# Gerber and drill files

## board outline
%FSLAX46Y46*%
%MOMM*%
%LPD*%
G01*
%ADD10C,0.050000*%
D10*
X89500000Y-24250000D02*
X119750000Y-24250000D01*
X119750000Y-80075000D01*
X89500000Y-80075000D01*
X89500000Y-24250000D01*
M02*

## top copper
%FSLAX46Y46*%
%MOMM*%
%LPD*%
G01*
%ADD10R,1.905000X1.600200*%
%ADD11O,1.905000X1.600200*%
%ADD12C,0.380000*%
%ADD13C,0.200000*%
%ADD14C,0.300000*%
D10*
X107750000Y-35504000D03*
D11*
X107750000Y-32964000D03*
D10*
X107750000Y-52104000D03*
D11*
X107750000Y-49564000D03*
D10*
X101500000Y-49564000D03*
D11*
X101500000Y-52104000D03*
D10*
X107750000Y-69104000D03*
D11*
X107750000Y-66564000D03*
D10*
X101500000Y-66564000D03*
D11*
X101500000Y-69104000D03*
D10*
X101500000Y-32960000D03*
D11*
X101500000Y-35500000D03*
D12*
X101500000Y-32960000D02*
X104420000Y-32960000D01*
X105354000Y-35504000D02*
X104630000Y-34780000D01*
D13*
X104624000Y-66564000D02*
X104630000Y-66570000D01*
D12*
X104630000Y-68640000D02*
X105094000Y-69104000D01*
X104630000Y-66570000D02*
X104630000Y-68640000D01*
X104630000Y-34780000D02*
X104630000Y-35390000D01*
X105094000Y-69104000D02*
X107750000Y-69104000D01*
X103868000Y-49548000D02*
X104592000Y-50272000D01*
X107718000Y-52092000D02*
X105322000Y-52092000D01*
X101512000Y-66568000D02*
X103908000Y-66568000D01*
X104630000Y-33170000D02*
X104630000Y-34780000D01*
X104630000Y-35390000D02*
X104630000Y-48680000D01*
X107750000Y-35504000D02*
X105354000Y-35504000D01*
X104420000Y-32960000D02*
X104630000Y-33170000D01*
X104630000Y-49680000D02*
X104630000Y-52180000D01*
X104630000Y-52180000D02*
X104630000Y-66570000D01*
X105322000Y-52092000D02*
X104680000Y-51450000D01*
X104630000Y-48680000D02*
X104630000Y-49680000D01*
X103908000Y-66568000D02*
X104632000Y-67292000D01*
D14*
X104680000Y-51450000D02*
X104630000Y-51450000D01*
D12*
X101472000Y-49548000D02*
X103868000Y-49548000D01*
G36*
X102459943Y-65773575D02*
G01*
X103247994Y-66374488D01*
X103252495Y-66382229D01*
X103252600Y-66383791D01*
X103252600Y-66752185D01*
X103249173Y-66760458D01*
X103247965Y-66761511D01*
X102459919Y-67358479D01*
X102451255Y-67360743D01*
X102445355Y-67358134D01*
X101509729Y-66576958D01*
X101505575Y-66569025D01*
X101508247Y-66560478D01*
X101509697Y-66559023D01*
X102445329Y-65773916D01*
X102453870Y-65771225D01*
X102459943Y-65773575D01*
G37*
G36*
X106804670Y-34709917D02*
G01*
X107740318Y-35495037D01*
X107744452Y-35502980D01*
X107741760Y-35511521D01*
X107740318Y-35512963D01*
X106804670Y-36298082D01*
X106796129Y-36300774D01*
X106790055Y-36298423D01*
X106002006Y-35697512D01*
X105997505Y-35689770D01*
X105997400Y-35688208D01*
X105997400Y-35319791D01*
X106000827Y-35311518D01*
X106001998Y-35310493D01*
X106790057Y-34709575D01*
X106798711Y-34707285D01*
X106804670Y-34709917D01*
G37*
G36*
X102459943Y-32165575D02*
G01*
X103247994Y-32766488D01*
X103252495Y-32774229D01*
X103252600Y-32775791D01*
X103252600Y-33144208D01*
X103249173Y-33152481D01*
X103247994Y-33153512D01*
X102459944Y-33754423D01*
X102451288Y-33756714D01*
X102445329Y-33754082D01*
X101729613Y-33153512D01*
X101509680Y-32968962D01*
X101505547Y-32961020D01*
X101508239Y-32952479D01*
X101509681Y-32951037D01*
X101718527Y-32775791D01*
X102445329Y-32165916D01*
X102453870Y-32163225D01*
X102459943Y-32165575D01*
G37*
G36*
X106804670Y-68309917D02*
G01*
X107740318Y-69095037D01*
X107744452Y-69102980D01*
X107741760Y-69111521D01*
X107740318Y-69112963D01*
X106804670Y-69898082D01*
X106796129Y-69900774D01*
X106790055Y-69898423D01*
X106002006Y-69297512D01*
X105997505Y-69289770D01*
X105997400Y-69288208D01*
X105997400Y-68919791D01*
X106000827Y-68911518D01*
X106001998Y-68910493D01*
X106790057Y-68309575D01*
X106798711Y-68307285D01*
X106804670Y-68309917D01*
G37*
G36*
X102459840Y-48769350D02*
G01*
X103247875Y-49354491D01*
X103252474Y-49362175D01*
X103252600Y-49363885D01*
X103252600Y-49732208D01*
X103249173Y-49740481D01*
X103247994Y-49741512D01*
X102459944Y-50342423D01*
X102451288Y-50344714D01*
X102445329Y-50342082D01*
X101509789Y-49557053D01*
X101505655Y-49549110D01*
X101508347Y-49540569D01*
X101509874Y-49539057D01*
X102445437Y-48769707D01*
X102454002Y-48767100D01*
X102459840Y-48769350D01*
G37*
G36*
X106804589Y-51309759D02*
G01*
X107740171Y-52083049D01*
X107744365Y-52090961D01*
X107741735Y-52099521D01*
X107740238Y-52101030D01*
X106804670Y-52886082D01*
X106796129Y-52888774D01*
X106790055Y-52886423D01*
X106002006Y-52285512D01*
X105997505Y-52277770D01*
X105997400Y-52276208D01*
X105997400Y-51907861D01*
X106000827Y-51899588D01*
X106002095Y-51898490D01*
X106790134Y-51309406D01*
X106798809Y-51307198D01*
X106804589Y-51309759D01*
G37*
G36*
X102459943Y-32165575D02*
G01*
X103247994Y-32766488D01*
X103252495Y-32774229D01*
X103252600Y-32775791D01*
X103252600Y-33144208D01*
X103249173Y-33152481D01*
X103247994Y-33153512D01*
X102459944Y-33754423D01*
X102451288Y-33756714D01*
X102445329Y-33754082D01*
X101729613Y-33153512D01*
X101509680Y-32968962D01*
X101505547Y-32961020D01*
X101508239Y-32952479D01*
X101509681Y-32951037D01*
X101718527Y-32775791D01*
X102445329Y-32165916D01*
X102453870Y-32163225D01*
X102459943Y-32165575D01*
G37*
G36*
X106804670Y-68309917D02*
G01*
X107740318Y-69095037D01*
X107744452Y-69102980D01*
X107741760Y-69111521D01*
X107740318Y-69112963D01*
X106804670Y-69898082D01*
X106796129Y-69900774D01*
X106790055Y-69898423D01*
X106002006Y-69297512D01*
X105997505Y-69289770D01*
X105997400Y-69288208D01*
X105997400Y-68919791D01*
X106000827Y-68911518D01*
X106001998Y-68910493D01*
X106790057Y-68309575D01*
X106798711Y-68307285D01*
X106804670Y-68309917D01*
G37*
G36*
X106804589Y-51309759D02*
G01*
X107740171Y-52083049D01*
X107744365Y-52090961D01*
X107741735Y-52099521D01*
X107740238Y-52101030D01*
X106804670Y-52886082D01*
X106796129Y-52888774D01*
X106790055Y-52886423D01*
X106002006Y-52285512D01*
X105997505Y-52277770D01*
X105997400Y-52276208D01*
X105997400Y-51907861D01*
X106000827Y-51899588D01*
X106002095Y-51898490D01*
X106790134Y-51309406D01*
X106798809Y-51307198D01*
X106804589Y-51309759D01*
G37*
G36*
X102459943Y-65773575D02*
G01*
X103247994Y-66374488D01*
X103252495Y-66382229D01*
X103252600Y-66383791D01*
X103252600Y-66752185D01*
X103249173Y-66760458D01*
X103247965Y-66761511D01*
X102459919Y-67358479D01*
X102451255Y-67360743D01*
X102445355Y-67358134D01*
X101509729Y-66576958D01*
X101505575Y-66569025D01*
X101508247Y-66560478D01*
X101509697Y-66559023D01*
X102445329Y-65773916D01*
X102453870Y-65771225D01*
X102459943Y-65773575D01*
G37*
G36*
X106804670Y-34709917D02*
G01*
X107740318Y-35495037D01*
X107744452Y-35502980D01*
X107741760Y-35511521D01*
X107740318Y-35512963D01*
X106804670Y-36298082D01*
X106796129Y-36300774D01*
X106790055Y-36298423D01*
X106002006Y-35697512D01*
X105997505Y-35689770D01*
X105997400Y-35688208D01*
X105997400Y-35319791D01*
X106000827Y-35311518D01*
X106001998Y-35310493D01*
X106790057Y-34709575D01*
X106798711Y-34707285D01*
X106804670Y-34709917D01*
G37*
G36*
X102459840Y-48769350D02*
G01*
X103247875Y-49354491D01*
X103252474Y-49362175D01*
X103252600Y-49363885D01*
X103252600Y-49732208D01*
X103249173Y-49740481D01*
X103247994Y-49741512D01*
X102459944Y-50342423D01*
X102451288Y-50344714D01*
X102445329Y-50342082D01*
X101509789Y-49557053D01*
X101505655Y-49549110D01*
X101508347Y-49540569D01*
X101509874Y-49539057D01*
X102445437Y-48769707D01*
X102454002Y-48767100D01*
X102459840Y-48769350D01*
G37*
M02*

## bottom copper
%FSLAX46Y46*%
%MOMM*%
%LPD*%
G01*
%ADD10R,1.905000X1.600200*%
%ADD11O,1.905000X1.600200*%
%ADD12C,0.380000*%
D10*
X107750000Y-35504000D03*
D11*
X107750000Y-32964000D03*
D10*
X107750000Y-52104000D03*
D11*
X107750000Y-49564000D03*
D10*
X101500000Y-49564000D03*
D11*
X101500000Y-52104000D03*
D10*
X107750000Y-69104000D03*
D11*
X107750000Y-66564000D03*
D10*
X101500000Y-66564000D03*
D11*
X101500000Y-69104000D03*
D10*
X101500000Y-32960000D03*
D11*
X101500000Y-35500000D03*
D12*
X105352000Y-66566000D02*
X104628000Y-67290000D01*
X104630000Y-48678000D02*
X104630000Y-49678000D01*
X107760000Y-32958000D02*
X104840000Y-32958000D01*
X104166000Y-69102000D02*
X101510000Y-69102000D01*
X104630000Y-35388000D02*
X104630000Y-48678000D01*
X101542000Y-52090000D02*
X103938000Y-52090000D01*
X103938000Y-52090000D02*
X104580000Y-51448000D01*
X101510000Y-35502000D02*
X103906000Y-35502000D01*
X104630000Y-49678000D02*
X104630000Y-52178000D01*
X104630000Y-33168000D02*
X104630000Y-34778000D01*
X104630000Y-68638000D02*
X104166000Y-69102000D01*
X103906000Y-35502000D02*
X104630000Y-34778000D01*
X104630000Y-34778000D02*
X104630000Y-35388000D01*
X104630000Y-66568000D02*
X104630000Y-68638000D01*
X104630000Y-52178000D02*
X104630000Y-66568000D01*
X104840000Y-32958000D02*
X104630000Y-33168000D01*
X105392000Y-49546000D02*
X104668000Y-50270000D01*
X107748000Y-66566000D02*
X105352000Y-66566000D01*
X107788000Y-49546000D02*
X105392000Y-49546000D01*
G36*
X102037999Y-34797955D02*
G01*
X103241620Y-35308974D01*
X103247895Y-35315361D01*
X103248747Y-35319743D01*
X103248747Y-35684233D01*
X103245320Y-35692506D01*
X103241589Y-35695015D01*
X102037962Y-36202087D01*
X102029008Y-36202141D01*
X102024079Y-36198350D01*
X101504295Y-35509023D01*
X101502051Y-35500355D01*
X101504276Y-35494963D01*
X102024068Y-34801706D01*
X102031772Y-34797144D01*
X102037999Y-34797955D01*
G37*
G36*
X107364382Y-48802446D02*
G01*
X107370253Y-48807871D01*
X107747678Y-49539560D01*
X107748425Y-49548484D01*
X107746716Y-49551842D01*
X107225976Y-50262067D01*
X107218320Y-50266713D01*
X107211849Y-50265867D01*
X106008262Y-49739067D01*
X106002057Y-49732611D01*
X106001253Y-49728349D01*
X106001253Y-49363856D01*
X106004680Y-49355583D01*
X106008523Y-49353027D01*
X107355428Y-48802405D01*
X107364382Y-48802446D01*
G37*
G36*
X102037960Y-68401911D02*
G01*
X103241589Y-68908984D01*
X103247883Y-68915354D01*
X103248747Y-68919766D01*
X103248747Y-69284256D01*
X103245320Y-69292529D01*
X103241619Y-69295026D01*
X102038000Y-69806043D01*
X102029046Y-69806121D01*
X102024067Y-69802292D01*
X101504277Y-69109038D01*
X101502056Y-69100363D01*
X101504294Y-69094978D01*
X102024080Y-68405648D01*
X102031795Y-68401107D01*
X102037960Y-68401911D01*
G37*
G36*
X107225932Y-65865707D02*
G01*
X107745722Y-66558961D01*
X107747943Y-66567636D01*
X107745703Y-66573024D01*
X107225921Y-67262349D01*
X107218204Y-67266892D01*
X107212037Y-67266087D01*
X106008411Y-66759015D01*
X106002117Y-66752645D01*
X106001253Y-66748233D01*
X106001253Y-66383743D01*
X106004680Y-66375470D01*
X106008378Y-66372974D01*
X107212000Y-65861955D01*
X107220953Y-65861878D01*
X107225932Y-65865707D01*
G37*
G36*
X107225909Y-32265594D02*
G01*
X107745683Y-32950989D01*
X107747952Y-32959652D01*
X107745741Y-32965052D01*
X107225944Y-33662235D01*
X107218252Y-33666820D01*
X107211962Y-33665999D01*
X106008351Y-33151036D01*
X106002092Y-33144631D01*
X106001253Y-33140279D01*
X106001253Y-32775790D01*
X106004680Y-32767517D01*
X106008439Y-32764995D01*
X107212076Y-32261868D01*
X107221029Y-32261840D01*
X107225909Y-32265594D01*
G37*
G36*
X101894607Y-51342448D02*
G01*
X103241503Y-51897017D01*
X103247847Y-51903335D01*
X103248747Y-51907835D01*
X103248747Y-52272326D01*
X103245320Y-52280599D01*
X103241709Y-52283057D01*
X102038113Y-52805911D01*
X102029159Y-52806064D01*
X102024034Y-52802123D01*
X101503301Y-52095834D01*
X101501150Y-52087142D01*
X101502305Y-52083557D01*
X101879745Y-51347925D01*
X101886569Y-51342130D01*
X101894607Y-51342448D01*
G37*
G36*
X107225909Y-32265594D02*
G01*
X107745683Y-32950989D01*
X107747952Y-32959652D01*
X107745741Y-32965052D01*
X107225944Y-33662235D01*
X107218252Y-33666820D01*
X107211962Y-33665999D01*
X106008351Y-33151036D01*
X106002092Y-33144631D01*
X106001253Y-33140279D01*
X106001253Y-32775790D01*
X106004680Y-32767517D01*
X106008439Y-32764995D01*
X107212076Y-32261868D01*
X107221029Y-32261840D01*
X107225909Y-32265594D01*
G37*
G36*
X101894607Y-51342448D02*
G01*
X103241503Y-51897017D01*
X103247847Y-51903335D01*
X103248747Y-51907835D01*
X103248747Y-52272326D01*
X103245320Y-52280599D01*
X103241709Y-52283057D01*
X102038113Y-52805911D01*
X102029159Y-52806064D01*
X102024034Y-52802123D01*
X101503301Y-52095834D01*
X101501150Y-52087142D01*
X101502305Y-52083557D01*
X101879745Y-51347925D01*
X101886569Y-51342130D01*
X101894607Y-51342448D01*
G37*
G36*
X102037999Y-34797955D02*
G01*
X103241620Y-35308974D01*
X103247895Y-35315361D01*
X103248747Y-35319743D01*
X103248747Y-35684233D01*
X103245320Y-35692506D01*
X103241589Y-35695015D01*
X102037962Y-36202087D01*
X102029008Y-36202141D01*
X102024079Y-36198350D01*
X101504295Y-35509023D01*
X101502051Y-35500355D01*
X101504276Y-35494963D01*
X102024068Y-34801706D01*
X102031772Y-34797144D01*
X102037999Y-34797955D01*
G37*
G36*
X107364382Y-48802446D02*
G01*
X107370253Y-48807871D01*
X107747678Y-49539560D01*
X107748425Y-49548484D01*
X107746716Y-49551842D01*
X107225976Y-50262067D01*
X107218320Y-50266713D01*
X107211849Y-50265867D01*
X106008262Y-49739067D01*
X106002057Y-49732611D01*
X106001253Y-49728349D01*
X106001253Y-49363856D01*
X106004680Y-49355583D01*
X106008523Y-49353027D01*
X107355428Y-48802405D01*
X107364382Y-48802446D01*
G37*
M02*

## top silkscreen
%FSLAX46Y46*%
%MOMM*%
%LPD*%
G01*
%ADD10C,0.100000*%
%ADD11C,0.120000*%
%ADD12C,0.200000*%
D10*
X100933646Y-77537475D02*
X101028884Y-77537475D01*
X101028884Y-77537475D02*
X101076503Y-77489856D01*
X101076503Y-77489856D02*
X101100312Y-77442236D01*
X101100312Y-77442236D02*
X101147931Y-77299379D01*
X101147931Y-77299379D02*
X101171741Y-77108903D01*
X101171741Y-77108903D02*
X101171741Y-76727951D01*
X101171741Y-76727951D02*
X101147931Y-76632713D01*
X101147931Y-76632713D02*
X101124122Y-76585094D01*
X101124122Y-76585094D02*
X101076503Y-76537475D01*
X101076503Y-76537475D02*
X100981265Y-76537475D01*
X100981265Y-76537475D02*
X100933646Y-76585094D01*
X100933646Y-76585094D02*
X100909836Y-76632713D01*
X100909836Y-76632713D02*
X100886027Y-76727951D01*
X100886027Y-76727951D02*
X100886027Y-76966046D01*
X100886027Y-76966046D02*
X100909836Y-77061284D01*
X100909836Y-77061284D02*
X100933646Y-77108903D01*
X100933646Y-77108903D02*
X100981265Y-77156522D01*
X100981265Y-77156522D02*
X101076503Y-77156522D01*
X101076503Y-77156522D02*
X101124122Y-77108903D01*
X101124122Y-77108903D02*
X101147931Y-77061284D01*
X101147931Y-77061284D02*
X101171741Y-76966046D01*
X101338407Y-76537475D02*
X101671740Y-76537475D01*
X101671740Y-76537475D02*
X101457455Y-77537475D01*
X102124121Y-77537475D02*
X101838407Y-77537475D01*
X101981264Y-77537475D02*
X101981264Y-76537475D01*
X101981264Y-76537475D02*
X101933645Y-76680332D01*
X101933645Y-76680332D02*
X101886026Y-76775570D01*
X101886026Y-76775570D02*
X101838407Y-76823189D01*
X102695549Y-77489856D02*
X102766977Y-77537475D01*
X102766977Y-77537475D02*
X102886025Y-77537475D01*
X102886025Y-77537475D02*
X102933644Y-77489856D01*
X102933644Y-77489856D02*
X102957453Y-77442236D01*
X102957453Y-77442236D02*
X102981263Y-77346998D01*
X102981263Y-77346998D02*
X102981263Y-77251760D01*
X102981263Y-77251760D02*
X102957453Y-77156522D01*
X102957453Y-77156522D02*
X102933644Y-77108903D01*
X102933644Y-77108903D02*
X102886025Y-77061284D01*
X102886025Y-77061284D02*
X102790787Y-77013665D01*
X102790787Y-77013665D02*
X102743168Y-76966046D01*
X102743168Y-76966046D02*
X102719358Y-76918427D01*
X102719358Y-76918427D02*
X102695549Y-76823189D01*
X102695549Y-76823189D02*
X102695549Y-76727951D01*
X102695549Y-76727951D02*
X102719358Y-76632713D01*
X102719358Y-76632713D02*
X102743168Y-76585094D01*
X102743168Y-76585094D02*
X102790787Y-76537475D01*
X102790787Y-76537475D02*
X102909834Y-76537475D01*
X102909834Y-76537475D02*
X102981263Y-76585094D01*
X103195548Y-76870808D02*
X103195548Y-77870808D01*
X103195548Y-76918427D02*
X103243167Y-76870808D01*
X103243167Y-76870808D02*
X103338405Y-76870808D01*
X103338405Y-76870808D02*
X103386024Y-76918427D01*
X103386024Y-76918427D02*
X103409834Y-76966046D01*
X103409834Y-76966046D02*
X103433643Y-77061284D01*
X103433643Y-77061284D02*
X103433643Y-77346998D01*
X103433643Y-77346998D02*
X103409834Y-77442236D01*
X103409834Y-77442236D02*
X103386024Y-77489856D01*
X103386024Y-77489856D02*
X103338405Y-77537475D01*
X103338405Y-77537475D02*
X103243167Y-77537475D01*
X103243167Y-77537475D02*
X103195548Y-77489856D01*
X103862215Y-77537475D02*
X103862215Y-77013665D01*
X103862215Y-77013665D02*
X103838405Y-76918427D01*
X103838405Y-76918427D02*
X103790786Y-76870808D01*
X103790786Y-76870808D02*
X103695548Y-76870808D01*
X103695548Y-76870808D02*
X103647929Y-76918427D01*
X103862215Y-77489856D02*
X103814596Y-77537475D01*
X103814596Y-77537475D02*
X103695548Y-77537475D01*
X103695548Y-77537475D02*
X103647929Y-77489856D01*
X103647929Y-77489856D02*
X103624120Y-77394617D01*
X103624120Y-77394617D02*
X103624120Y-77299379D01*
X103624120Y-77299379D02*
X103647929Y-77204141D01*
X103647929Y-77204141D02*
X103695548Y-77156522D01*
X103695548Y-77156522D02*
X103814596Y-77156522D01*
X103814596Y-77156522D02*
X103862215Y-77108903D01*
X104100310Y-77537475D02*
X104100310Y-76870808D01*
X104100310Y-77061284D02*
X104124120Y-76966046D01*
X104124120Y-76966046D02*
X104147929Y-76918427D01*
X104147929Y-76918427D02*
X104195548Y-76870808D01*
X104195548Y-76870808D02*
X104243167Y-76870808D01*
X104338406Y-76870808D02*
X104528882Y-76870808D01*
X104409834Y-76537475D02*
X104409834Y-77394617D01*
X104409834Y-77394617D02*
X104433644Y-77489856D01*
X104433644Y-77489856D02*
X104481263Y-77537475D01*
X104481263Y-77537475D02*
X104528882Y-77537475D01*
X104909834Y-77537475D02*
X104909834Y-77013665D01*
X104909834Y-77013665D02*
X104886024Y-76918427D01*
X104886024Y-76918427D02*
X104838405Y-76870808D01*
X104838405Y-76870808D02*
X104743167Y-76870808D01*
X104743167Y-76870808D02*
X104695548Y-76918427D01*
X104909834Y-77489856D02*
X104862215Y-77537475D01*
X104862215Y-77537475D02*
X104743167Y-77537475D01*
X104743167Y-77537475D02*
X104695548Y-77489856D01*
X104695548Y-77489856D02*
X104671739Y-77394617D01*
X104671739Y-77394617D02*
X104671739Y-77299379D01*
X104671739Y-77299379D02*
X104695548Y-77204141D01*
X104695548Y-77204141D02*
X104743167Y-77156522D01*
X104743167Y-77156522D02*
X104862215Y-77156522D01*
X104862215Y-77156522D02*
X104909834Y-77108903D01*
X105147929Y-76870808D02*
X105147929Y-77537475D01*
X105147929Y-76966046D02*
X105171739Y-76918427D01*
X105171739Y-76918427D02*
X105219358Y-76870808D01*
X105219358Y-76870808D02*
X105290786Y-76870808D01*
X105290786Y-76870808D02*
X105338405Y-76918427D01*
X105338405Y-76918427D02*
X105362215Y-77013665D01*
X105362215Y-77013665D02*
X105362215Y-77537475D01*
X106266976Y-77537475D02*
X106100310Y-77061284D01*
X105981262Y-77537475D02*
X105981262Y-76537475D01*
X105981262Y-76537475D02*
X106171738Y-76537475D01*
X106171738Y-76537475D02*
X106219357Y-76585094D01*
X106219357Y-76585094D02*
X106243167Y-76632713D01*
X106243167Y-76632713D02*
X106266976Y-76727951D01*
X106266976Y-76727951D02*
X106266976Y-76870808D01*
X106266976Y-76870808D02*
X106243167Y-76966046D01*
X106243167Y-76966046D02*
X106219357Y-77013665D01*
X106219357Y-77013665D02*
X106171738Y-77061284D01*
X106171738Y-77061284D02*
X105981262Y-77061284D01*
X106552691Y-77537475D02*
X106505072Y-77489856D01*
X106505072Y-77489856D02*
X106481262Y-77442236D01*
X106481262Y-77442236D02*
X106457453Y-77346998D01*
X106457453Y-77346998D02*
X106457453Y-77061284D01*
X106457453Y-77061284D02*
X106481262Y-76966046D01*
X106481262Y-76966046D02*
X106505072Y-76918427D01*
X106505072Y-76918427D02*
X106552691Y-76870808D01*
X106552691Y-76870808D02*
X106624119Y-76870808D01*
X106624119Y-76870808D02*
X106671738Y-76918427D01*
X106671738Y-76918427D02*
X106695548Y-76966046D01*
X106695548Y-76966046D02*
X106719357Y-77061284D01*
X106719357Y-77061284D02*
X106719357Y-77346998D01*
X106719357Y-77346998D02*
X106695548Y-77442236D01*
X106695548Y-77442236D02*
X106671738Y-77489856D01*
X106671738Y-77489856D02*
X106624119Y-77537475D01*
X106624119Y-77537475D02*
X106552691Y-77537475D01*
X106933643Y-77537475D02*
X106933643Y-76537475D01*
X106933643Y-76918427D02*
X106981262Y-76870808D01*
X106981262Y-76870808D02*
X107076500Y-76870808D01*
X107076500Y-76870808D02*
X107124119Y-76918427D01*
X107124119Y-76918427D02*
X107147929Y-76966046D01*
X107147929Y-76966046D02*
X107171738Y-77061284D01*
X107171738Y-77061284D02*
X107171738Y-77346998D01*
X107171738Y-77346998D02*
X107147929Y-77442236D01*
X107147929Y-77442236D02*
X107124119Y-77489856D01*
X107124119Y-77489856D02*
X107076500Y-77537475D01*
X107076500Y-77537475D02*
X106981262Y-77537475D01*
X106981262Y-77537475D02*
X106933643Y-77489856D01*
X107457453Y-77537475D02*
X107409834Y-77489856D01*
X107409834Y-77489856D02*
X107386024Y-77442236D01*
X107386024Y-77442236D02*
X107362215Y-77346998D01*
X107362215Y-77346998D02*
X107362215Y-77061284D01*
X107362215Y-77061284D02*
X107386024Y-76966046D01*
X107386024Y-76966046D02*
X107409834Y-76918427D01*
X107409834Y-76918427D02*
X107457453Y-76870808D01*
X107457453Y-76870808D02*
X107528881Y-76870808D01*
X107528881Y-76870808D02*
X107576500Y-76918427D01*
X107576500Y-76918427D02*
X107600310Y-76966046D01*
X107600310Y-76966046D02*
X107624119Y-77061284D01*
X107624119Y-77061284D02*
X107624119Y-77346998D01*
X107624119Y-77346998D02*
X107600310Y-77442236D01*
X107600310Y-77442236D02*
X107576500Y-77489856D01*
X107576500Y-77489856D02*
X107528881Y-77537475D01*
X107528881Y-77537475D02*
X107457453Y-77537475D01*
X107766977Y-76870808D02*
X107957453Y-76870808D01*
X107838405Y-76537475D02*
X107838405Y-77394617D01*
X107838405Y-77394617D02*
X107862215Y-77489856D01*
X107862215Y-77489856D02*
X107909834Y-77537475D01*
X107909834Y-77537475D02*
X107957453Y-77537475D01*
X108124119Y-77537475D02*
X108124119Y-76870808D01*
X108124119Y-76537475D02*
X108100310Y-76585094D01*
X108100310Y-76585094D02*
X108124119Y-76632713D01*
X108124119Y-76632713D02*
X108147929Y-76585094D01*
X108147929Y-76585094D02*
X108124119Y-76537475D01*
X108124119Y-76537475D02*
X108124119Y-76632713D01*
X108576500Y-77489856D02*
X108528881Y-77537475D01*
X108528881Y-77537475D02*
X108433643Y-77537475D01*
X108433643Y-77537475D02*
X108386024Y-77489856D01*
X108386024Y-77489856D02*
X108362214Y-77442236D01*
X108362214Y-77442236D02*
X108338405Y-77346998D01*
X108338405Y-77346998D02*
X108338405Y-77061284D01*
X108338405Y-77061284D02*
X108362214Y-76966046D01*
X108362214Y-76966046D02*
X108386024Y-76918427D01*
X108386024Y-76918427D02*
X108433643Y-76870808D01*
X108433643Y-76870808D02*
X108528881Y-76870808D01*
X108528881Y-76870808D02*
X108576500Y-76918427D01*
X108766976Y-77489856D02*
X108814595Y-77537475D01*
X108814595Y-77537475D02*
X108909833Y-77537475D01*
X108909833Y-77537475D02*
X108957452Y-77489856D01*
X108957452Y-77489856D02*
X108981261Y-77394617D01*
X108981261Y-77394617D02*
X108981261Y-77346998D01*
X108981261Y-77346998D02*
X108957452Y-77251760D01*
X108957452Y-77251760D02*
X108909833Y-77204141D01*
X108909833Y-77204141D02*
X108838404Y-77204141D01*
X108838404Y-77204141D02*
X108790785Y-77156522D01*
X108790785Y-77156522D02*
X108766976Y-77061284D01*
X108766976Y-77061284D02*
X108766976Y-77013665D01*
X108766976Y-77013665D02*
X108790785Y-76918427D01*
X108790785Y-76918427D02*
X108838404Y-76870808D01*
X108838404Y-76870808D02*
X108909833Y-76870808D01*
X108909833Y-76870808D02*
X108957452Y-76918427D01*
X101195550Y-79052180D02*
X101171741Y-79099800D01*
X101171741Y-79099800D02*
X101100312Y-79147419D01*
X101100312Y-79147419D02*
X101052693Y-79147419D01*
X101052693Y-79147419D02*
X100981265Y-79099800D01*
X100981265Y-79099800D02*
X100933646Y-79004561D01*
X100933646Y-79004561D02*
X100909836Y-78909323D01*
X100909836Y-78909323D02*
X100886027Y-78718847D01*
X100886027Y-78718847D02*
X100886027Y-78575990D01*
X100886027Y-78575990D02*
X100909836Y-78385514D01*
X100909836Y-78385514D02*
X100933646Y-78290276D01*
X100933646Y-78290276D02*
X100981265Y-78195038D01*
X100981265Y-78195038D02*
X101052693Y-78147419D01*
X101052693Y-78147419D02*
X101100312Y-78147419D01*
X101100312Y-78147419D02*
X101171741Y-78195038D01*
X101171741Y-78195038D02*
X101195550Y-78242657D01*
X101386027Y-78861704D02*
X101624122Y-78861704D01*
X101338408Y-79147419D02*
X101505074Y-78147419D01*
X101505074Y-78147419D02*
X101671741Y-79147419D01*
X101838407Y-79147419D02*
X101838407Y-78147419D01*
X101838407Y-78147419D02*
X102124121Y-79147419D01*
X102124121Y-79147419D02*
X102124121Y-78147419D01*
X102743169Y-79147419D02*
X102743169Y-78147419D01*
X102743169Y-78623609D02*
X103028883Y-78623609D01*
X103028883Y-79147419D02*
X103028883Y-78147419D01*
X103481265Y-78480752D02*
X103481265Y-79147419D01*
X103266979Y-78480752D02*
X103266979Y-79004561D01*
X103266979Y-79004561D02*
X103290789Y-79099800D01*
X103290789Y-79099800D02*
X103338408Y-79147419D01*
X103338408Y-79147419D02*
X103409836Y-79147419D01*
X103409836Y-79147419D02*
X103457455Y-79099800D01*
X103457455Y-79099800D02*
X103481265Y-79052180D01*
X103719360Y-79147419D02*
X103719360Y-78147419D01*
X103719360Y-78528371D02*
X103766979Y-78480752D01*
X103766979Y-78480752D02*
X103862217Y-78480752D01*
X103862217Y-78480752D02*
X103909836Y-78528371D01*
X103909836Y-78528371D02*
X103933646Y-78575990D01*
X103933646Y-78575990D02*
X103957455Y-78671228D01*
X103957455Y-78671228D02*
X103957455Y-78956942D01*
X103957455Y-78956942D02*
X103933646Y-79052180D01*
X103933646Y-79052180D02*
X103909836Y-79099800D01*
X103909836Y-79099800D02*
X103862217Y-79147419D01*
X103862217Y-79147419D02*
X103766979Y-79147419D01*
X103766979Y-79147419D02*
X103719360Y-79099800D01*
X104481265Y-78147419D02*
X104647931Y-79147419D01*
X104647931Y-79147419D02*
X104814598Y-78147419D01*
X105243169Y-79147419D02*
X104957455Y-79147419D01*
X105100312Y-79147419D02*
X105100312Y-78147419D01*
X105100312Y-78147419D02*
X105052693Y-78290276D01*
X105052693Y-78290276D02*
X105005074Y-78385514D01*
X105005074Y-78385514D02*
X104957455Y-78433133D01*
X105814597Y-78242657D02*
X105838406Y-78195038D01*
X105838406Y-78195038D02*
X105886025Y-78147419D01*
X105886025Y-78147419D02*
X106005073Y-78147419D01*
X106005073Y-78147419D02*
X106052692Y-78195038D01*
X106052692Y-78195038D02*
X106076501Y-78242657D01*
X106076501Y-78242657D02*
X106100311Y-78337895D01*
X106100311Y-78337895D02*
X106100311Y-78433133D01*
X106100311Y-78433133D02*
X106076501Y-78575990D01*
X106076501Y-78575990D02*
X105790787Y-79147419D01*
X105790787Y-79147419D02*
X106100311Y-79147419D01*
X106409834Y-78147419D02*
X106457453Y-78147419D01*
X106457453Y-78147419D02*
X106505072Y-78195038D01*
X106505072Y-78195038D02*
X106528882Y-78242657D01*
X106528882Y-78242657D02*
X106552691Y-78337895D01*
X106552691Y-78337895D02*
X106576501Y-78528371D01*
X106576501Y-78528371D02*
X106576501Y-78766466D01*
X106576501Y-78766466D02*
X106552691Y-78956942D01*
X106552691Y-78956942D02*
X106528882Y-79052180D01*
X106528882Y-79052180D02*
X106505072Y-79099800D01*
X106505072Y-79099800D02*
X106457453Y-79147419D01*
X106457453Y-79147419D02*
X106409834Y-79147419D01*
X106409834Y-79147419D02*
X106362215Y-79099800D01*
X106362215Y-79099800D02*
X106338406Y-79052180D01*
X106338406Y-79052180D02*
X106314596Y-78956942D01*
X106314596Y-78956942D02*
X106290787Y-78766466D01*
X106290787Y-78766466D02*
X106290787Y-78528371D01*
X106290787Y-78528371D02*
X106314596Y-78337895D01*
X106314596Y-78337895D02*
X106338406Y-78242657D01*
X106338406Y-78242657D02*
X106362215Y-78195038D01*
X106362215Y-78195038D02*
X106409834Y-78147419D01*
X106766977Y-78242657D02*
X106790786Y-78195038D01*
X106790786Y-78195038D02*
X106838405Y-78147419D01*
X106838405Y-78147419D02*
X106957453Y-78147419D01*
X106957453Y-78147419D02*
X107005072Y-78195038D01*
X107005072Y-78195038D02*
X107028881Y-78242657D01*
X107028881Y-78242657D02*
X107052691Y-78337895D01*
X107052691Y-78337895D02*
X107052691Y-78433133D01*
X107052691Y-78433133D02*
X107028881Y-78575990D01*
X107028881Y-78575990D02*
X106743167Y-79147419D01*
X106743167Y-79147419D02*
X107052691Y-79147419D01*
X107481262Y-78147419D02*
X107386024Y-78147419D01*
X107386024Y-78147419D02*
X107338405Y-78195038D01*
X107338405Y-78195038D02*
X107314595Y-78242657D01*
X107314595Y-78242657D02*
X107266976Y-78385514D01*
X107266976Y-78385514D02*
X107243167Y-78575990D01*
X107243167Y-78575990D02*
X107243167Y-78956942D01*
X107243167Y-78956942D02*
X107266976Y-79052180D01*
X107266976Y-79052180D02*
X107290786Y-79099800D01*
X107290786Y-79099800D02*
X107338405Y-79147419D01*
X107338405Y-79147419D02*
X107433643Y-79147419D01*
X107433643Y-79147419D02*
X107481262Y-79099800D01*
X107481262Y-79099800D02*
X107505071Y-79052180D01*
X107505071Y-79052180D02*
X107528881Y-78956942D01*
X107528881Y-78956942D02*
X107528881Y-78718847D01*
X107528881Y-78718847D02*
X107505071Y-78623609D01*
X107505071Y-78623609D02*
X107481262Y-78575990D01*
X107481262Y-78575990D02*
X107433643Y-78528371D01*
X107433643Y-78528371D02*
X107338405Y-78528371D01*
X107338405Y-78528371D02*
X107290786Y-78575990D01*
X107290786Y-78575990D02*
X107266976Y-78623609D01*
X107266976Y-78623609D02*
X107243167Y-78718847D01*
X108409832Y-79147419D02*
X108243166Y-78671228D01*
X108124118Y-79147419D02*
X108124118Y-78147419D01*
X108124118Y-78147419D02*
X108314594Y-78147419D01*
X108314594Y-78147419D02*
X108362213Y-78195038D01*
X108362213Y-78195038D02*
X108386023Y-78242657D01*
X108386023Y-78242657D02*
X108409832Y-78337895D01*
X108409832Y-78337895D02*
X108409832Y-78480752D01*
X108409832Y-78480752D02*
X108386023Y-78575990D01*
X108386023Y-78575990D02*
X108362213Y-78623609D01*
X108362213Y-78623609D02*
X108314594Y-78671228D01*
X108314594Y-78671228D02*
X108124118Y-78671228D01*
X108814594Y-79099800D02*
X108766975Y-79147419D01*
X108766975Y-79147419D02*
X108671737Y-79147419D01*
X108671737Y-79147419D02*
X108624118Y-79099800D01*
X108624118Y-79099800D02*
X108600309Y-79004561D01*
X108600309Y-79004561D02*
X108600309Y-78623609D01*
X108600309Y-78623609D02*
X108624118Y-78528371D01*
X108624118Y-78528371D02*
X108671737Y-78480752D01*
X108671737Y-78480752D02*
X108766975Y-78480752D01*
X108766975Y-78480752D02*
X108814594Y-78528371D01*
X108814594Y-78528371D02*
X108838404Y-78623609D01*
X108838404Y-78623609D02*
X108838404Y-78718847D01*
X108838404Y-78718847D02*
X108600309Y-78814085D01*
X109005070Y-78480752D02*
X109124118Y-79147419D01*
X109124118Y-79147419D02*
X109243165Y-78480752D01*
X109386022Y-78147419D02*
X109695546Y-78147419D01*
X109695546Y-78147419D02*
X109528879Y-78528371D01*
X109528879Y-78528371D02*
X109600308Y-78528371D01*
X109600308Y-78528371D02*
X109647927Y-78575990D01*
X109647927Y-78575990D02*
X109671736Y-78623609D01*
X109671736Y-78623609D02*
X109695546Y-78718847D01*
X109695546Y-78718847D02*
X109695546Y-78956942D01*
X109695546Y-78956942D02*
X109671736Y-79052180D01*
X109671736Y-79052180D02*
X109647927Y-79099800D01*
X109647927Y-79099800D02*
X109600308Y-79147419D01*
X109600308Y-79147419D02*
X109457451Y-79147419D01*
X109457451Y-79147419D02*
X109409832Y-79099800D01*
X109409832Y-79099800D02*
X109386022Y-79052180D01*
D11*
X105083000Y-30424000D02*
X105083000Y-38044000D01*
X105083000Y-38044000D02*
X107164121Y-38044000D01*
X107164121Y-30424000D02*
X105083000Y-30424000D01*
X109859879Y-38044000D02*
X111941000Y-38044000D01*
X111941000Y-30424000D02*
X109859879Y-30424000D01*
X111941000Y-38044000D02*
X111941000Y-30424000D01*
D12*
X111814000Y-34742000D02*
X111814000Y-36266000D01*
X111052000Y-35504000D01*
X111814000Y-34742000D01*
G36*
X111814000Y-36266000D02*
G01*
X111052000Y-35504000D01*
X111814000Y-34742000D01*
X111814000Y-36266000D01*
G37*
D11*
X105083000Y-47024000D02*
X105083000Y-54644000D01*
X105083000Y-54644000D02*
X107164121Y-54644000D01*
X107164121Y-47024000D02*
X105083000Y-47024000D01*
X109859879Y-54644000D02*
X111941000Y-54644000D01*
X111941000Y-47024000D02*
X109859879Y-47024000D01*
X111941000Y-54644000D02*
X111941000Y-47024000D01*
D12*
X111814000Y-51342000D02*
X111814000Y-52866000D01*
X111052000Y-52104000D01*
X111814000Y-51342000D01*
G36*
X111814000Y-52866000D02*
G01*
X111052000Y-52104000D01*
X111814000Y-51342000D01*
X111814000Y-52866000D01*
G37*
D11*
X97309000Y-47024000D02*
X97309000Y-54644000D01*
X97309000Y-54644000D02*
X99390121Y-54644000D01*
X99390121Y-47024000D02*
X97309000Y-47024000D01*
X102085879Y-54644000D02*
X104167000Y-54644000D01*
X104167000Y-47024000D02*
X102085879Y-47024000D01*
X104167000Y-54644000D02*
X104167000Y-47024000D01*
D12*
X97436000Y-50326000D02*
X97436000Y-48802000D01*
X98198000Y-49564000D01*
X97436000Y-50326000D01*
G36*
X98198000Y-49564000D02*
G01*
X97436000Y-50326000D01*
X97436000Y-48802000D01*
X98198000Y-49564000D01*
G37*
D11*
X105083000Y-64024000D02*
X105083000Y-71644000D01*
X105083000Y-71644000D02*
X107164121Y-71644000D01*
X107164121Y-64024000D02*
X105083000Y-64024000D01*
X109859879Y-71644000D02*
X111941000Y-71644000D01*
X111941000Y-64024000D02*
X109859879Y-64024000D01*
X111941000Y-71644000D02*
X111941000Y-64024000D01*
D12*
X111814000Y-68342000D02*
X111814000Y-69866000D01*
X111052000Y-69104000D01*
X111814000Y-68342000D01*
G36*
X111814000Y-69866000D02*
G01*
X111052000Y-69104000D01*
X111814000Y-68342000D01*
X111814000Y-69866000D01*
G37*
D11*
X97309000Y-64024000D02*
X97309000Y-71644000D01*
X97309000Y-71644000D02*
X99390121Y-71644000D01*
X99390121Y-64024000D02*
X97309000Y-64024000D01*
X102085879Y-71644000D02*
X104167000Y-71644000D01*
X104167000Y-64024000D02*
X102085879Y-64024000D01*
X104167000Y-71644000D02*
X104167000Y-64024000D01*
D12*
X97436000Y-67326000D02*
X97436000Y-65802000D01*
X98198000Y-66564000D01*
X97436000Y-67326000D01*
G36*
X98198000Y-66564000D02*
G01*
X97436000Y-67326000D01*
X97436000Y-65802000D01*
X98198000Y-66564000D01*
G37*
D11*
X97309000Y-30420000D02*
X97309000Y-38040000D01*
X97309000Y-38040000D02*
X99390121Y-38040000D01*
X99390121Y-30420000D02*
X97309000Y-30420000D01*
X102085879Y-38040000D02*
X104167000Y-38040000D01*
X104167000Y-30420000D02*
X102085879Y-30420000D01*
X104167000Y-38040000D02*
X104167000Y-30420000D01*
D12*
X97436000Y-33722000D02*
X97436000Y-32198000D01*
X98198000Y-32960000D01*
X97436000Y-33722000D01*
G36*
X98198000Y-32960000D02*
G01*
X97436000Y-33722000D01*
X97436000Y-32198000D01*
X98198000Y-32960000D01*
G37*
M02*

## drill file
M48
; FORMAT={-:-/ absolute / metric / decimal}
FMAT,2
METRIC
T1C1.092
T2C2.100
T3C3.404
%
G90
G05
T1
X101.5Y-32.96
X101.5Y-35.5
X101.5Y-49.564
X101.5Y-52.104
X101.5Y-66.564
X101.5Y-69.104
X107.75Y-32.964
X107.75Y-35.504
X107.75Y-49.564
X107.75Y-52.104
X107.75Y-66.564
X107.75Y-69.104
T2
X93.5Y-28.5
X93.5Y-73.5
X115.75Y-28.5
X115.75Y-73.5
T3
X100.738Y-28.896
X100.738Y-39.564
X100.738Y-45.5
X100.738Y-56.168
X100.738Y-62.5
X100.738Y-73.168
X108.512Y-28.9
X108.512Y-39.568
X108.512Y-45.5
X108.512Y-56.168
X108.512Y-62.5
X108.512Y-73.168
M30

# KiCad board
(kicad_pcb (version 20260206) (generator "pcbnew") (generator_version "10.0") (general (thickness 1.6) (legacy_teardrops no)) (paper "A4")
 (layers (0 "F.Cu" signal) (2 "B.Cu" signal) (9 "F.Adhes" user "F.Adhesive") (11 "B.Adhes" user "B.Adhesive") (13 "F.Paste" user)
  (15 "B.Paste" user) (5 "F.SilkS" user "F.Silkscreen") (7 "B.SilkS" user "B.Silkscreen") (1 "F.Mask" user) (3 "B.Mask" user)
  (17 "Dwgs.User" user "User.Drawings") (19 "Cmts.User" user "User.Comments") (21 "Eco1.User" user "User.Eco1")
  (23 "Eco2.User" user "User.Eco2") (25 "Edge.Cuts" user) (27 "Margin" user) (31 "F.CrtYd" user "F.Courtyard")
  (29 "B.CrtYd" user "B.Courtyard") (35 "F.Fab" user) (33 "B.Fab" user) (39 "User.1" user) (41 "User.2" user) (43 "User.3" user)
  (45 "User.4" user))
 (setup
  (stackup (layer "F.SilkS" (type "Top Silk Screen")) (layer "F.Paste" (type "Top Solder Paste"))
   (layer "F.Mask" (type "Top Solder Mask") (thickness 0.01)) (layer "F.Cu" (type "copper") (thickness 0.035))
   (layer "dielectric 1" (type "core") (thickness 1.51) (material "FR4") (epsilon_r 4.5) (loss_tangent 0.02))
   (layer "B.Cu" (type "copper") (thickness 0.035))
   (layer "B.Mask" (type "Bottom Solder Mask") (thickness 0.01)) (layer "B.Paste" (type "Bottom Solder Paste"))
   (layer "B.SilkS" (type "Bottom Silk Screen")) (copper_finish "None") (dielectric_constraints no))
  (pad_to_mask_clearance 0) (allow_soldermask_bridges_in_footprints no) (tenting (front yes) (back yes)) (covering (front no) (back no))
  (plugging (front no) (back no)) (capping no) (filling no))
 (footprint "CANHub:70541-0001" (layer "F.Cu") (at 107.75 35.504 90)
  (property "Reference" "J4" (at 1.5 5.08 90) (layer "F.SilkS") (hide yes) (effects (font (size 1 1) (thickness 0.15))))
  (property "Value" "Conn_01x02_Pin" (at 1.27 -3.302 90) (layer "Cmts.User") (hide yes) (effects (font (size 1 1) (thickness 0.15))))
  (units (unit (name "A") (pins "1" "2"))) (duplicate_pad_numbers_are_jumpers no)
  (fp_line (start 5.08 -2.667) (end -2.54 -2.667) (stroke (width 0.12) (type solid)) (layer "F.SilkS"))
  (fp_line (start -2.54 -2.667) (end -2.54 -0.585879) (stroke (width 0.12) (type solid)) (layer "F.SilkS"))
  (fp_line (start 5.08 -0.585879) (end 5.08 -2.667) (stroke (width 0.12) (type solid)) (layer "F.SilkS"))
  (fp_line (start -2.54 2.109879) (end -2.54 4.191) (stroke (width 0.12) (type solid)) (layer "F.SilkS"))
  (fp_line (start 5.08 4.191) (end 5.08 2.109879) (stroke (width 0.12) (type solid)) (layer "F.SilkS"))
  (fp_line (start -2.54 4.191) (end 5.08 4.191) (stroke (width 0.12) (type solid)) (layer "F.SilkS"))
  (fp_poly (pts (xy 0.762 4.064) (xy -0.762 4.064) (xy 0 3.302)) (stroke (width 0.2) (type solid)) (fill yes) (layer "F.SilkS"))
  (pad "" np_thru_hole circle (at -4.064 0.762 90) (size 3.4036 3.4036) (drill 3.4036) (layers "*.Cu" "*.Mask"))
  (pad "" np_thru_hole circle (at 6.604 0.762 90) (size 3.4036 3.4036) (drill 3.4036) (layers "*.Cu" "*.Mask"))
  (pad "1" thru_hole rect (at 0 0 90) (size 1.6002 1.905) (drill 1.0922) (layers "*.Cu" "*.Mask") (remove_unused_layers no) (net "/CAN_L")
   (teardrops (best_length_ratio 0.5) (max_length 1) (best_width_ratio 1) (max_width 2) (curved_edges no) (filter_ratio 0.9) (enabled yes)
    (allow_two_segments yes) (prefer_zone_connections yes)))
  (pad "2" thru_hole oval (at 2.54 0 90) (size 1.6002 1.905) (drill 1.0922) (layers "*.Cu" "*.Mask") (remove_unused_layers no)
   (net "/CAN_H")
   (teardrops (best_length_ratio 0.5) (max_length 1) (best_width_ratio 1) (max_width 2) (curved_edges no) (filter_ratio 0.9) (enabled yes)
    (allow_two_segments yes) (prefer_zone_connections yes))))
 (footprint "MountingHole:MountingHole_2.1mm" (layer "F.Cu") (at 93.5 73.5)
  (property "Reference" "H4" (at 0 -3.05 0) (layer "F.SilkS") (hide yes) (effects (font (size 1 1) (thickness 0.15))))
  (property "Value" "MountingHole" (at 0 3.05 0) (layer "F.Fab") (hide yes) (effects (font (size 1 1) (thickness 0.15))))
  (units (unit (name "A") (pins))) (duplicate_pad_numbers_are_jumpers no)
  (pad "" np_thru_hole circle (at 0 0) (size 2.1 2.1) (drill 2.1) (layers "*.Cu" "*.Mask")))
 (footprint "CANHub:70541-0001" (layer "F.Cu") (at 107.75 52.104 90)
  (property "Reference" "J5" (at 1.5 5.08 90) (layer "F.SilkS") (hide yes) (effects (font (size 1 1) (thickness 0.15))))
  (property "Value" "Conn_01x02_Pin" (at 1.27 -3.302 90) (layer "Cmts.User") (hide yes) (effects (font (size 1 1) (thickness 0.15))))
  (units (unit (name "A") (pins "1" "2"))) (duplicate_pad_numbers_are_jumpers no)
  (fp_line (start 5.08 -2.667) (end -2.54 -2.667) (stroke (width 0.12) (type solid)) (layer "F.SilkS"))
  (fp_line (start -2.54 -2.667) (end -2.54 -0.585879) (stroke (width 0.12) (type solid)) (layer "F.SilkS"))
  (fp_line (start 5.08 -0.585879) (end 5.08 -2.667) (stroke (width 0.12) (type solid)) (layer "F.SilkS"))
  (fp_line (start -2.54 2.109879) (end -2.54 4.191) (stroke (width 0.12) (type solid)) (layer "F.SilkS"))
  (fp_line (start 5.08 4.191) (end 5.08 2.109879) (stroke (width 0.12) (type solid)) (layer "F.SilkS"))
  (fp_line (start -2.54 4.191) (end 5.08 4.191) (stroke (width 0.12) (type solid)) (layer "F.SilkS"))
  (fp_poly (pts (xy 0.762 4.064) (xy -0.762 4.064) (xy 0 3.302)) (stroke (width 0.2) (type solid)) (fill yes) (layer "F.SilkS"))
  (pad "" np_thru_hole circle (at -4.064 0.762 90) (size 3.4036 3.4036) (drill 3.4036) (layers "*.Cu" "*.Mask"))
  (pad "" np_thru_hole circle (at 6.604 0.762 90) (size 3.4036 3.4036) (drill 3.4036) (layers "*.Cu" "*.Mask"))
  (pad "1" thru_hole rect (at 0 0 90) (size 1.6002 1.905) (drill 1.0922) (layers "*.Cu" "*.Mask") (remove_unused_layers no) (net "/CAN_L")
   (teardrops (best_length_ratio 0.5) (max_length 1) (best_width_ratio 1) (max_width 2) (curved_edges no) (filter_ratio 0.9) (enabled yes)
    (allow_two_segments yes) (prefer_zone_connections yes)))
  (pad "2" thru_hole oval (at 2.54 0 90) (size 1.6002 1.905) (drill 1.0922) (layers "*.Cu" "*.Mask") (remove_unused_layers no)
   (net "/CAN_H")
   (teardrops (best_length_ratio 0.5) (max_length 1) (best_width_ratio 1) (max_width 2) (curved_edges no) (filter_ratio 0.9) (enabled yes)
    (allow_two_segments yes) (prefer_zone_connections yes))))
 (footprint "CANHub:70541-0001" (layer "F.Cu") (at 101.5 49.564 -90)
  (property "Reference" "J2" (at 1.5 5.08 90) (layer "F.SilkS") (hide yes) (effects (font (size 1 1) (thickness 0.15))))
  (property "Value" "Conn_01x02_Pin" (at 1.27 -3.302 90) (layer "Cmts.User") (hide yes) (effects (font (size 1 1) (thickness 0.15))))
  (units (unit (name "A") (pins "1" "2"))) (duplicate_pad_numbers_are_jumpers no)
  (fp_line (start -2.54 4.191) (end 5.08 4.191) (stroke (width 0.12) (type solid)) (layer "F.SilkS"))
  (fp_line (start 5.08 4.191) (end 5.08 2.109879) (stroke (width 0.12) (type solid)) (layer "F.SilkS"))
  (fp_line (start -2.54 2.109879) (end -2.54 4.191) (stroke (width 0.12) (type solid)) (layer "F.SilkS"))
  (fp_line (start 5.08 -0.585879) (end 5.08 -2.667) (stroke (width 0.12) (type solid)) (layer "F.SilkS"))
  (fp_line (start -2.54 -2.667) (end -2.54 -0.585879) (stroke (width 0.12) (type solid)) (layer "F.SilkS"))
  (fp_line (start 5.08 -2.667) (end -2.54 -2.667) (stroke (width 0.12) (type solid)) (layer "F.SilkS"))
  (fp_poly (pts (xy 0.762 4.064) (xy -0.762 4.064) (xy 0 3.302)) (stroke (width 0.2) (type solid)) (fill yes) (layer "F.SilkS"))
  (pad "" np_thru_hole circle (at -4.064 0.762 270) (size 3.4036 3.4036) (drill 3.4036) (layers "*.Cu" "*.Mask"))
  (pad "" np_thru_hole circle (at 6.604 0.762 270) (size 3.4036 3.4036) (drill 3.4036) (layers "*.Cu" "*.Mask"))
  (pad "1" thru_hole rect (at 0 0 270) (size 1.6002 1.905) (drill 1.0922) (layers "*.Cu" "*.Mask") (remove_unused_layers no) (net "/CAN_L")
   (teardrops (best_length_ratio 0.5) (max_length 1) (best_width_ratio 1) (max_width 2) (curved_edges no) (filter_ratio 0.9) (enabled yes)
    (allow_two_segments yes) (prefer_zone_connections yes)))
  (pad "2" thru_hole oval (at 2.54 0 270) (size 1.6002 1.905) (drill 1.0922) (layers "*.Cu" "*.Mask") (remove_unused_layers no)
   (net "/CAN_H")
   (teardrops (best_length_ratio 0.5) (max_length 1) (best_width_ratio 1) (max_width 2) (curved_edges no) (filter_ratio 0.9) (enabled yes)
    (allow_two_segments yes) (prefer_zone_connections yes))))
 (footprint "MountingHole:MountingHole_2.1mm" (layer "F.Cu") (at 115.75 73.5)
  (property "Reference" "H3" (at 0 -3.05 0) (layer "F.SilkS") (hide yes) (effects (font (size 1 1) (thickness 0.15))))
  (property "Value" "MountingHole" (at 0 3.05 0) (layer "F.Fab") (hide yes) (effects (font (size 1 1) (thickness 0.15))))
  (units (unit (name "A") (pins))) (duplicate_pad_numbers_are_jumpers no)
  (pad "" np_thru_hole circle (at 0 0) (size 2.1 2.1) (drill 2.1) (layers "*.Cu" "*.Mask")))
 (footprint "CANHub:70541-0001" (layer "F.Cu") (at 107.75 69.104 90)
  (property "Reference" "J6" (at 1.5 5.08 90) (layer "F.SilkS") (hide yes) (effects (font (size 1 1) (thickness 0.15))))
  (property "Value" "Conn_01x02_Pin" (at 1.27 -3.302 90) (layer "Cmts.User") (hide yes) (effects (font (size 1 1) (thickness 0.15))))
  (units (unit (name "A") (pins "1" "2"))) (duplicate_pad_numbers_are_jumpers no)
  (fp_line (start 5.08 -2.667) (end -2.54 -2.667) (stroke (width 0.12) (type solid)) (layer "F.SilkS"))
  (fp_line (start -2.54 -2.667) (end -2.54 -0.585879) (stroke (width 0.12) (type solid)) (layer "F.SilkS"))
  (fp_line (start 5.08 -0.585879) (end 5.08 -2.667) (stroke (width 0.12) (type solid)) (layer "F.SilkS"))
  (fp_line (start -2.54 2.109879) (end -2.54 4.191) (stroke (width 0.12) (type solid)) (layer "F.SilkS"))
  (fp_line (start 5.08 4.191) (end 5.08 2.109879) (stroke (width 0.12) (type solid)) (layer "F.SilkS"))
  (fp_line (start -2.54 4.191) (end 5.08 4.191) (stroke (width 0.12) (type solid)) (layer "F.SilkS"))
  (fp_poly (pts (xy 0.762 4.064) (xy -0.762 4.064) (xy 0 3.302)) (stroke (width 0.2) (type solid)) (fill yes) (layer "F.SilkS"))
  (pad "" np_thru_hole circle (at -4.064 0.762 90) (size 3.4036 3.4036) (drill 3.4036) (layers "*.Cu" "*.Mask"))
  (pad "" np_thru_hole circle (at 6.604 0.762 90) (size 3.4036 3.4036) (drill 3.4036) (layers "*.Cu" "*.Mask"))
  (pad "1" thru_hole rect (at 0 0 90) (size 1.6002 1.905) (drill 1.0922) (layers "*.Cu" "*.Mask") (remove_unused_layers no) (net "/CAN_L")
   (teardrops (best_length_ratio 0.5) (max_length 1) (best_width_ratio 1) (max_width 2) (curved_edges no) (filter_ratio 0.9) (enabled yes)
    (allow_two_segments yes) (prefer_zone_connections yes)))
  (pad "2" thru_hole oval (at 2.54 0 90) (size 1.6002 1.905) (drill 1.0922) (layers "*.Cu" "*.Mask") (remove_unused_layers no)
   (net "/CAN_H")
   (teardrops (best_length_ratio 0.5) (max_length 1) (best_width_ratio 1) (max_width 2) (curved_edges no) (filter_ratio 0.9) (enabled yes)
    (allow_two_segments yes) (prefer_zone_connections yes))))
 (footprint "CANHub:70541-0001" (layer "F.Cu") (at 101.5 66.564 -90)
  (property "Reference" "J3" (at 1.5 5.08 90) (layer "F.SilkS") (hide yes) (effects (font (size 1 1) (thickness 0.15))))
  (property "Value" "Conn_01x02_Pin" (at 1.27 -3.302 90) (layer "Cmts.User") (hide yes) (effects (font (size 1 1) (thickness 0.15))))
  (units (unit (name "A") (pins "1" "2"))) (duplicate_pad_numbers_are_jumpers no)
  (fp_line (start -2.54 4.191) (end 5.08 4.191) (stroke (width 0.12) (type solid)) (layer "F.SilkS"))
  (fp_line (start 5.08 4.191) (end 5.08 2.109879) (stroke (width 0.12) (type solid)) (layer "F.SilkS"))
  (fp_line (start -2.54 2.109879) (end -2.54 4.191) (stroke (width 0.12) (type solid)) (layer "F.SilkS"))
  (fp_line (start 5.08 -0.585879) (end 5.08 -2.667) (stroke (width 0.12) (type solid)) (layer "F.SilkS"))
  (fp_line (start -2.54 -2.667) (end -2.54 -0.585879) (stroke (width 0.12) (type solid)) (layer "F.SilkS"))
  (fp_line (start 5.08 -2.667) (end -2.54 -2.667) (stroke (width 0.12) (type solid)) (layer "F.SilkS"))
  (fp_poly (pts (xy 0.762 4.064) (xy -0.762 4.064) (xy 0 3.302)) (stroke (width 0.2) (type solid)) (fill yes) (layer "F.SilkS"))
  (pad "" np_thru_hole circle (at -4.064 0.762 270) (size 3.4036 3.4036) (drill 3.4036) (layers "*.Cu" "*.Mask"))
  (pad "" np_thru_hole circle (at 6.604 0.762 270) (size 3.4036 3.4036) (drill 3.4036) (layers "*.Cu" "*.Mask"))
  (pad "1" thru_hole rect (at 0 0 270) (size 1.6002 1.905) (drill 1.0922) (layers "*.Cu" "*.Mask") (remove_unused_layers no) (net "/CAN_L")
   (teardrops (best_length_ratio 0.5) (max_length 1) (best_width_ratio 1) (max_width 2) (curved_edges no) (filter_ratio 0.9) (enabled yes)
    (allow_two_segments yes) (prefer_zone_connections yes)))
  (pad "2" thru_hole oval (at 2.54 0 270) (size 1.6002 1.905) (drill 1.0922) (layers "*.Cu" "*.Mask") (remove_unused_layers no)
   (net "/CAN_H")
   (teardrops (best_length_ratio 0.5) (max_length 1) (best_width_ratio 1) (max_width 2) (curved_edges no) (filter_ratio 0.9) (enabled yes)
    (allow_two_segments yes) (prefer_zone_connections yes))))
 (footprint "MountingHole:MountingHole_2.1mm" (layer "F.Cu") (at 93.5 28.5)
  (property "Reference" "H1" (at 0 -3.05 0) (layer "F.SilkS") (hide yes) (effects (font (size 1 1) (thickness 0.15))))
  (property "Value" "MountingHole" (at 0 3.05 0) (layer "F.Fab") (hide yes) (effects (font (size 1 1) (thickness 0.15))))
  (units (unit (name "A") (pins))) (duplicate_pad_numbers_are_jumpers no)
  (pad "" np_thru_hole circle (at 0 0) (size 2.1 2.1) (drill 2.1) (layers "*.Cu" "*.Mask")))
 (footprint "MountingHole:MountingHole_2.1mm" (layer "F.Cu") (at 115.75 28.5)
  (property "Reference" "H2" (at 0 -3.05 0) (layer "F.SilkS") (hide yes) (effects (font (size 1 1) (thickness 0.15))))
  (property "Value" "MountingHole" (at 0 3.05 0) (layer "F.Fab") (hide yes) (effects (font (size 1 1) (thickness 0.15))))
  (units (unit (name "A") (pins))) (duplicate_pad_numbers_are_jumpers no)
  (pad "" np_thru_hole circle (at 0 0) (size 2.1 2.1) (drill 2.1) (layers "*.Cu" "*.Mask")))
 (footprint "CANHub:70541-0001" (layer "F.Cu") (at 101.5 32.96 -90)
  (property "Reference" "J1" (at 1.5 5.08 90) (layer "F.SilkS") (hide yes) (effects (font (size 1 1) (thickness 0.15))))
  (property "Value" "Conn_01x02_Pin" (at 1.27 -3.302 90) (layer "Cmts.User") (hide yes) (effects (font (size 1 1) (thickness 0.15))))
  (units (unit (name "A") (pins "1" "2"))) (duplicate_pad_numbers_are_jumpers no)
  (fp_line (start -2.54 4.191) (end 5.08 4.191) (stroke (width 0.12) (type solid)) (layer "F.SilkS"))
  (fp_line (start 5.08 4.191) (end 5.08 2.109879) (stroke (width 0.12) (type solid)) (layer "F.SilkS"))
  (fp_line (start -2.54 2.109879) (end -2.54 4.191) (stroke (width 0.12) (type solid)) (layer "F.SilkS"))
  (fp_line (start 5.08 -0.585879) (end 5.08 -2.667) (stroke (width 0.12) (type solid)) (layer "F.SilkS"))
  (fp_line (start -2.54 -2.667) (end -2.54 -0.585879) (stroke (width 0.12) (type solid)) (layer "F.SilkS"))
  (fp_line (start 5.08 -2.667) (end -2.54 -2.667) (stroke (width 0.12) (type solid)) (layer "F.SilkS"))
  (fp_poly (pts (xy 0.762 4.064) (xy -0.762 4.064) (xy 0 3.302)) (stroke (width 0.2) (type solid)) (fill yes) (layer "F.SilkS"))
  (pad "" np_thru_hole circle (at -4.064 0.762 270) (size 3.4036 3.4036) (drill 3.4036) (layers "*.Cu" "*.Mask"))
  (pad "" np_thru_hole circle (at 6.604 0.762 270) (size 3.4036 3.4036) (drill 3.4036) (layers "*.Cu" "*.Mask"))
  (pad "1" thru_hole rect (at 0 0 270) (size 1.6002 1.905) (drill 1.0922) (layers "*.Cu" "*.Mask") (remove_unused_layers no) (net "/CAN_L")
   (teardrops (best_length_ratio 0.5) (max_length 1) (best_width_ratio 1) (max_width 2) (curved_edges no) (filter_ratio 0.9) (enabled yes)
    (allow_two_segments yes) (prefer_zone_connections yes)))
  (pad "2" thru_hole oval (at 2.54 0 270) (size 1.6002 1.905) (drill 1.0922) (layers "*.Cu" "*.Mask") (remove_unused_layers no)
   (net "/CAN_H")
   (teardrops (best_length_ratio 0.5) (max_length 1) (best_width_ratio 1) (max_width 2) (curved_edges no) (filter_ratio 0.9) (enabled yes)
    (allow_two_segments yes) (prefer_zone_connections yes))))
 (gr_rect (start 89.5 24.25) (end 119.75 80.075) (stroke (width 0.05) (type default)) (fill no) (layer "Edge.Cuts"))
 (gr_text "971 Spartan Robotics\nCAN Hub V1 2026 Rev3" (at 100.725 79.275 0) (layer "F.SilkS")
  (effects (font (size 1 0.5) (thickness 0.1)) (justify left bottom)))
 (segment (start 101.5 32.96) (end 104.42 32.96) (width 0.38) (layer "F.Cu") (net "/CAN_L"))
 (segment (start 105.354 35.504) (end 104.63 34.78) (width 0.38) (layer "F.Cu") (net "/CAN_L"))
 (segment (start 104.624 66.564) (end 104.63 66.57) (width 0.2) (layer "F.Cu") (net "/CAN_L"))
 (segment (start 104.63 68.64) (end 105.094 69.104) (width 0.38) (layer "F.Cu") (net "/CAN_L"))
 (segment (start 104.63 66.57) (end 104.63 68.64) (width 0.38) (layer "F.Cu") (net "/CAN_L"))
 (segment (start 104.63 34.78) (end 104.63 35.39) (width 0.38) (layer "F.Cu") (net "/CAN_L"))
 (segment (start 105.094 69.104) (end 107.75 69.104) (width 0.38) (layer "F.Cu") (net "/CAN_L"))
 (segment (start 103.868 49.548) (end 104.592 50.272) (width 0.38) (layer "F.Cu") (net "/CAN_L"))
 (segment (start 107.718 52.092) (end 105.322 52.092) (width 0.38) (layer "F.Cu") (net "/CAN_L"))
 (segment (start 101.512 66.568) (end 103.908 66.568) (width 0.38) (layer "F.Cu") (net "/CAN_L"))
 (segment (start 104.63 33.17) (end 104.63 34.78) (width 0.38) (layer "F.Cu") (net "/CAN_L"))
 (segment (start 104.63 35.39) (end 104.63 48.68) (width 0.38) (layer "F.Cu") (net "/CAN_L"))
 (segment (start 107.75 35.504) (end 105.354 35.504) (width 0.38) (layer "F.Cu") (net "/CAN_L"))
 (segment (start 104.42 32.96) (end 104.63 33.17) (width 0.38) (layer "F.Cu") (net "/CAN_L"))
 (segment (start 104.63 49.68) (end 104.63 52.18) (width 0.38) (layer "F.Cu") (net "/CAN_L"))
 (segment (start 104.63 52.18) (end 104.63 66.57) (width 0.38) (layer "F.Cu") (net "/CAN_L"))
 (segment (start 105.322 52.092) (end 104.68 51.45) (width 0.38) (layer "F.Cu") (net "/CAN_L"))
 (segment (start 104.63 48.68) (end 104.63 49.68) (width 0.38) (layer "F.Cu") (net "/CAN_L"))
 (segment (start 103.908 66.568) (end 104.632 67.292) (width 0.38) (layer "F.Cu") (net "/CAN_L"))
 (segment (start 104.68 51.45) (end 104.63 51.45) (width 0.3) (layer "F.Cu") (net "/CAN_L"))
 (segment (start 101.472 49.548) (end 103.868 49.548) (width 0.38) (layer "F.Cu") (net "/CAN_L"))
 (segment (start 105.352 66.566) (end 104.628 67.29) (width 0.38) (layer "B.Cu") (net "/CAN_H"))
 (segment (start 104.63 48.678) (end 104.63 49.678) (width 0.38) (layer "B.Cu") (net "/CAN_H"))
 (segment (start 107.76 32.958) (end 104.84 32.958) (width 0.38) (layer "B.Cu") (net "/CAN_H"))
 (segment (start 104.166 69.102) (end 101.51 69.102) (width 0.38) (layer "B.Cu") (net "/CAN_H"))
 (segment (start 104.63 35.388) (end 104.63 48.678) (width 0.38) (layer "B.Cu") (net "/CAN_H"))
 (segment (start 101.542 52.09) (end 103.938 52.09) (width 0.38) (layer "B.Cu") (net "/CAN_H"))
 (segment (start 103.938 52.09) (end 104.58 51.448) (width 0.38) (layer "B.Cu") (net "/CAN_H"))
 (segment (start 101.51 35.502) (end 103.906 35.502) (width 0.38) (layer "B.Cu") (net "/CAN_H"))
 (segment (start 104.63 49.678) (end 104.63 52.178) (width 0.38) (layer "B.Cu") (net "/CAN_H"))
 (segment (start 104.63 33.168) (end 104.63 34.778) (width 0.38) (layer "B.Cu") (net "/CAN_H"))
 (segment (start 104.63 68.638) (end 104.166 69.102) (width 0.38) (layer "B.Cu") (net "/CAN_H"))
 (segment (start 103.906 35.502) (end 104.63 34.778) (width 0.38) (layer "B.Cu") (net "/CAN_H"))
 (segment (start 104.63 34.778) (end 104.63 35.388) (width 0.38) (layer "B.Cu") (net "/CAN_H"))
 (segment (start 104.63 66.568) (end 104.63 68.638) (width 0.38) (layer "B.Cu") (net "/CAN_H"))
 (segment (start 104.63 52.178) (end 104.63 66.568) (width 0.38) (layer "B.Cu") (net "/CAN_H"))
 (segment (start 104.84 32.958) (end 104.63 33.168) (width 0.38) (layer "B.Cu") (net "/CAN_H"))
 (segment (start 105.392 49.546) (end 104.668 50.27) (width 0.38) (layer "B.Cu") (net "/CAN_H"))
 (segment (start 107.748 66.566) (end 105.352 66.566) (width 0.38) (layer "B.Cu") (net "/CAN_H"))
 (segment (start 107.788 49.546) (end 105.392 49.546) (width 0.38) (layer "B.Cu") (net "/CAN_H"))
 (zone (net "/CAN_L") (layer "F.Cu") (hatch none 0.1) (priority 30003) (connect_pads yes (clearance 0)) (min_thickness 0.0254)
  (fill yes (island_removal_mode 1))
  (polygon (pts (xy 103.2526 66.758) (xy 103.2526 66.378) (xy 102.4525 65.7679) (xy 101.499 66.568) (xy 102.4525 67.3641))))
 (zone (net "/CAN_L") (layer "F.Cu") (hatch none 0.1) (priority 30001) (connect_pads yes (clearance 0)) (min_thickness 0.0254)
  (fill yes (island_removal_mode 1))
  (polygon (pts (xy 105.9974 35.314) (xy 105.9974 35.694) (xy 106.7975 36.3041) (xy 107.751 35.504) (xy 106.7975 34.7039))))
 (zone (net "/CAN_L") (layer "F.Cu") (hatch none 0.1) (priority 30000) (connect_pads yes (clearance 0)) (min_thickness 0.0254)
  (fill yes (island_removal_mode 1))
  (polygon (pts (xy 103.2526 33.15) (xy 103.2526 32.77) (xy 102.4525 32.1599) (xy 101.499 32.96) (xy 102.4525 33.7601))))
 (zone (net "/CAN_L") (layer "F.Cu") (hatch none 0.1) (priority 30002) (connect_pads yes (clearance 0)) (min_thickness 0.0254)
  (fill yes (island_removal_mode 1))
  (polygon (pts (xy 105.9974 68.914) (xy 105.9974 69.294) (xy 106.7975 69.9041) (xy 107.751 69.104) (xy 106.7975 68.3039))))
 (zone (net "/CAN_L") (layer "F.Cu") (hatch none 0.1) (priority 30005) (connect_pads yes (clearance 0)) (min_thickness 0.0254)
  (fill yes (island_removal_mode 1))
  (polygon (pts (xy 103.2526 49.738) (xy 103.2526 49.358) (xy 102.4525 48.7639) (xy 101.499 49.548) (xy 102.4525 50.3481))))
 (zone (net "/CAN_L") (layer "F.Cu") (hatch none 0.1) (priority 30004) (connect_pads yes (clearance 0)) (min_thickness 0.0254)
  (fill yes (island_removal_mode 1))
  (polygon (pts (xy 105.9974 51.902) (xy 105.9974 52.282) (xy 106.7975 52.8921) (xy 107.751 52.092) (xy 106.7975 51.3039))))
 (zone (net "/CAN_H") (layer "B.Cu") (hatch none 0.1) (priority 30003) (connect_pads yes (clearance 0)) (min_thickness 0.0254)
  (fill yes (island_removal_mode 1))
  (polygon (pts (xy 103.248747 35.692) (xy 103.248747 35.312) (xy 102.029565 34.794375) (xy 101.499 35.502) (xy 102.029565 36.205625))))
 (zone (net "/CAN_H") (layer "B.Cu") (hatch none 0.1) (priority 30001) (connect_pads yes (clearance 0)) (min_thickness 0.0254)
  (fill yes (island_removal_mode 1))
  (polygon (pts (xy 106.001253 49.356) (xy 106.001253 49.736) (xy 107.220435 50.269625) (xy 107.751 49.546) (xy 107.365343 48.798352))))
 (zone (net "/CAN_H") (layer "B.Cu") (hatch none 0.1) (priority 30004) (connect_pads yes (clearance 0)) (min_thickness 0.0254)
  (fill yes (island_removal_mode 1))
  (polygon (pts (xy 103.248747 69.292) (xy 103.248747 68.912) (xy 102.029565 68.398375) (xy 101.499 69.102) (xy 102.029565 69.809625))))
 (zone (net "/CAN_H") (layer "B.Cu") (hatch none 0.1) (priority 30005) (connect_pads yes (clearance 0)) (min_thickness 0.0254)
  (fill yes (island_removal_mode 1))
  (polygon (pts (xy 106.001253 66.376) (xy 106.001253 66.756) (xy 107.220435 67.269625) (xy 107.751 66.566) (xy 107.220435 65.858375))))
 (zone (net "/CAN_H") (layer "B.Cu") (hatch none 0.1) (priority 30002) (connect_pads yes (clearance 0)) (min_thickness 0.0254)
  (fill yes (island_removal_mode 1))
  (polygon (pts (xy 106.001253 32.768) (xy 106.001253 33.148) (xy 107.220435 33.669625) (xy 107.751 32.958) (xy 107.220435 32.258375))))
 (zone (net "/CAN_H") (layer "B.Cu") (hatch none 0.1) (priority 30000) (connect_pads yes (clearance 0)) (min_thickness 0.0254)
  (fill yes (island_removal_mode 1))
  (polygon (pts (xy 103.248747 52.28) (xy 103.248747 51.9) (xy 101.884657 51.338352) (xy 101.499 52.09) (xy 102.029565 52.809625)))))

